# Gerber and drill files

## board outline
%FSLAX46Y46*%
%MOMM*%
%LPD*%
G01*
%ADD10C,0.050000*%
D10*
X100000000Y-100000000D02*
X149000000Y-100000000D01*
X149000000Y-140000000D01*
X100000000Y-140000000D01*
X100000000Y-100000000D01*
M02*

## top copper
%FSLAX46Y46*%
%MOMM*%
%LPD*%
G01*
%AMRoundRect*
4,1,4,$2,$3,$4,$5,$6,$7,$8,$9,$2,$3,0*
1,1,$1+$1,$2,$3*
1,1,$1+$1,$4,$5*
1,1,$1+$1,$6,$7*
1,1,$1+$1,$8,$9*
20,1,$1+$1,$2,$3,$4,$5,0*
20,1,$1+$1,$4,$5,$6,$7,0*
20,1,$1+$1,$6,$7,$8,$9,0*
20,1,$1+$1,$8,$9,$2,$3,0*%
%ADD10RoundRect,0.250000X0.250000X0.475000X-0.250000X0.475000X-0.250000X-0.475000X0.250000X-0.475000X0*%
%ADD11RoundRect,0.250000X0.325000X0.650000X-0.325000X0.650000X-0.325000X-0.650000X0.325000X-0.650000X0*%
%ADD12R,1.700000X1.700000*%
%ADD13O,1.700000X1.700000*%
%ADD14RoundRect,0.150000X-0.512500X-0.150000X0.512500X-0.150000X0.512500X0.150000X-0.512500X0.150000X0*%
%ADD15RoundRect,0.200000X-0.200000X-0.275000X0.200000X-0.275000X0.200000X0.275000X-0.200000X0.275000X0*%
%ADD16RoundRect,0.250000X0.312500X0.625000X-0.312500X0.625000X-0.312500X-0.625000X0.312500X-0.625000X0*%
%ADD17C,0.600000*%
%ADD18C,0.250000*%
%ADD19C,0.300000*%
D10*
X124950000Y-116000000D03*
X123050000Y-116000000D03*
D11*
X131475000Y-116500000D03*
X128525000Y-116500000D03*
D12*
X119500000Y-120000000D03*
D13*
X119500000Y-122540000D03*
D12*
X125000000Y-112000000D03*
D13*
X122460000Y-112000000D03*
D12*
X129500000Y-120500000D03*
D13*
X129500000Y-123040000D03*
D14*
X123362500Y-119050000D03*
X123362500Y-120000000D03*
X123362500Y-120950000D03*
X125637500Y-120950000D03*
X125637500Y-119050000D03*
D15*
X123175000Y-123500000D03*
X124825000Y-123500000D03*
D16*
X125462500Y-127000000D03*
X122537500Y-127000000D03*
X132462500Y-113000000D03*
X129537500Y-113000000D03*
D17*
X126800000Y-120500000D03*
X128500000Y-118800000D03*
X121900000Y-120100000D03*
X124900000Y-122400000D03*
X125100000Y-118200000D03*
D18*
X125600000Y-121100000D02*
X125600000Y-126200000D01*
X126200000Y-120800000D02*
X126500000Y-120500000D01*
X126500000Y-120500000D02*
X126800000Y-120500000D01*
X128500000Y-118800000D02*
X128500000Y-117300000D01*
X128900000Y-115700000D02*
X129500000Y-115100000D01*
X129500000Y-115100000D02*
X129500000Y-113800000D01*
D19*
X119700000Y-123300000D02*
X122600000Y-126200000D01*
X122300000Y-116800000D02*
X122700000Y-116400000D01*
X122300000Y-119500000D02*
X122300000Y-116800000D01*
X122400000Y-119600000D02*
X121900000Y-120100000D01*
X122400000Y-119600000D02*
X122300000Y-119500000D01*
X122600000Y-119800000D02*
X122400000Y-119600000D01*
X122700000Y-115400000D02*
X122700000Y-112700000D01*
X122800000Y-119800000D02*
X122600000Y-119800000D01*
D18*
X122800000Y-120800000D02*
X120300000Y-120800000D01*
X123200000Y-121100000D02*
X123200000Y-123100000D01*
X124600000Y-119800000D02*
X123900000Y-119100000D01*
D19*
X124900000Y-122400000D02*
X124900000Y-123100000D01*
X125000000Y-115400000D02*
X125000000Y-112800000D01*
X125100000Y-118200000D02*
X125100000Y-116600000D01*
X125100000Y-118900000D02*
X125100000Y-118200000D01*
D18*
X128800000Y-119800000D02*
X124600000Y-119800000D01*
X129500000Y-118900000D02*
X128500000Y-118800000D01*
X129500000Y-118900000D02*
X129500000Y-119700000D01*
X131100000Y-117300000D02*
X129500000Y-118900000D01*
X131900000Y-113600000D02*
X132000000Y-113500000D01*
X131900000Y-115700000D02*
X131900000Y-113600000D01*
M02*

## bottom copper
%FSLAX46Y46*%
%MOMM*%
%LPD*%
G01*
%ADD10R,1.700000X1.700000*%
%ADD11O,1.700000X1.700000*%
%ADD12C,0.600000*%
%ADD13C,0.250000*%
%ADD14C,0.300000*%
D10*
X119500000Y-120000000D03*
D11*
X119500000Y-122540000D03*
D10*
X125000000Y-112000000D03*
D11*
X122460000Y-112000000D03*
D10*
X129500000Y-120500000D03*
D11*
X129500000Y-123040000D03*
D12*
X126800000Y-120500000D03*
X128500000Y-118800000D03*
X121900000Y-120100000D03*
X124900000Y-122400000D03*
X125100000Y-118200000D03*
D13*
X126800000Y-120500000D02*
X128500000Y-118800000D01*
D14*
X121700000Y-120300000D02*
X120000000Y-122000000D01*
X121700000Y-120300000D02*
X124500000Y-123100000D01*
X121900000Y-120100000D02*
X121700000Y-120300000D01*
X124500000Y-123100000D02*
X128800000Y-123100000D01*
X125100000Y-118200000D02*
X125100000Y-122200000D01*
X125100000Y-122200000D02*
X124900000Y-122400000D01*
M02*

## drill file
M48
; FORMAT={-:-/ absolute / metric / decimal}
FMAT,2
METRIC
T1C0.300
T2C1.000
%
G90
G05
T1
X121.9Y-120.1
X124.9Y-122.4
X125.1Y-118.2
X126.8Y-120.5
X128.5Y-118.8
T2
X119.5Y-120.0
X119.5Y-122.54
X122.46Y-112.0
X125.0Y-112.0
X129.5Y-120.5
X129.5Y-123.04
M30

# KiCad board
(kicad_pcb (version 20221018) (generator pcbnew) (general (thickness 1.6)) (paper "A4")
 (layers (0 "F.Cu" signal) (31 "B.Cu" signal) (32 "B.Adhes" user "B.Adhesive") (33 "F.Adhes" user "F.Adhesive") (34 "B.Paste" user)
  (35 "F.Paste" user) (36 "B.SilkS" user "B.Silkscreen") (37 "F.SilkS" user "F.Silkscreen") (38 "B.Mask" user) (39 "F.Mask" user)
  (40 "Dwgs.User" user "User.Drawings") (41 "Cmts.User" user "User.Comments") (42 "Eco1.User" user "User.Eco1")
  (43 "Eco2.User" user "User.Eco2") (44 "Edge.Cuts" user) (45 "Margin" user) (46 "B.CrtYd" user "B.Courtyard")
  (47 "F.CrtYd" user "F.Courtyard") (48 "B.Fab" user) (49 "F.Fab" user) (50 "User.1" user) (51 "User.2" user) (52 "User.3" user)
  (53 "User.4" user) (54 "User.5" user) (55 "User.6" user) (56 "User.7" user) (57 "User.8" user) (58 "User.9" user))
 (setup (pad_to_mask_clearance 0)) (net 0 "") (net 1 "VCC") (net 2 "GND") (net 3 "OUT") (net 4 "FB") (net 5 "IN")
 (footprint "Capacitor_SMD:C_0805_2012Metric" (layer "F.Cu") (at 124 116 180)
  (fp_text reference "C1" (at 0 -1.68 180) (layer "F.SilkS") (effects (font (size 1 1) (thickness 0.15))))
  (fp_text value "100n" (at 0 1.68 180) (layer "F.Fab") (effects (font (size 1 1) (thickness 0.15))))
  (pad "1" smd roundrect (at -0.95 0 180) (size 1 1.45) (layers "F.Cu" "F.Paste" "F.Mask") (roundrect_rratio 0.25) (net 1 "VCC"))
  (pad "2" smd roundrect (at 0.95 0 180) (size 1 1.45) (layers "F.Cu" "F.Paste" "F.Mask") (roundrect_rratio 0.25) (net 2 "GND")))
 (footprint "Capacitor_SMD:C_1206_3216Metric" (layer "F.Cu") (at 130 116.5 180)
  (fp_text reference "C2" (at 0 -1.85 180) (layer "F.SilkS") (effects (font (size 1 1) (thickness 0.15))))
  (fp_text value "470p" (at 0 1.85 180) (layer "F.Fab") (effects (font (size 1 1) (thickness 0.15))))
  (pad "1" smd roundrect (at -1.475 0 180) (size 1.15 1.8) (layers "F.Cu" "F.Paste" "F.Mask") (roundrect_rratio 0.217391) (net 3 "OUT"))
  (pad "2" smd roundrect (at 1.475 0 180) (size 1.15 1.8) (layers "F.Cu" "F.Paste" "F.Mask") (roundrect_rratio 0.217391) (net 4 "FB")))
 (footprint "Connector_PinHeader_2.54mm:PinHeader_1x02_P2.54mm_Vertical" (layer "F.Cu") (at 119.5 120)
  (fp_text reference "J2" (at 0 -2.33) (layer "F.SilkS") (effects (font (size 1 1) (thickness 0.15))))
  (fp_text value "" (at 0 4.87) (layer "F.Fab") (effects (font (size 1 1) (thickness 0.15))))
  (pad "1" thru_hole rect (at 0 0) (size 1.7 1.7) (drill 1) (layers "*.Cu" "*.Mask") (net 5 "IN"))
  (pad "2" thru_hole oval (at 0 2.54) (size 1.7 1.7) (drill 1) (layers "*.Cu" "*.Mask") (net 2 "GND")))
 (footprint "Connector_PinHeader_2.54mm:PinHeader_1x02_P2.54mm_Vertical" (layer "F.Cu") (at 125 112 -90)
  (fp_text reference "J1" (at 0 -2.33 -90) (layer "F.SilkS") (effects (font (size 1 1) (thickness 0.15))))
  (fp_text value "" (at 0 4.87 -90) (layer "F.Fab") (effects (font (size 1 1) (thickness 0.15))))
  (pad "1" thru_hole rect (at 0 0 270) (size 1.7 1.7) (drill 1) (layers "*.Cu" "*.Mask") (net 1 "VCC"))
  (pad "2" thru_hole oval (at 0 2.54 270) (size 1.7 1.7) (drill 1) (layers "*.Cu" "*.Mask") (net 2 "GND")))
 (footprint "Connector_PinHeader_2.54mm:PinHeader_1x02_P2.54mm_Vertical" (layer "F.Cu") (at 129.5 120.5)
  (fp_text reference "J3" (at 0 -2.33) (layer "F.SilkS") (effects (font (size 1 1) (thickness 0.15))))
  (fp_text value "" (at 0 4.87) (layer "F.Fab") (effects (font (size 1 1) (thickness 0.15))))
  (pad "1" thru_hole rect (at 0 0) (size 1.7 1.7) (drill 1) (layers "*.Cu" "*.Mask") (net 3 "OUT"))
  (pad "2" thru_hole oval (at 0 2.54) (size 1.7 1.7) (drill 1) (layers "*.Cu" "*.Mask") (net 2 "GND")))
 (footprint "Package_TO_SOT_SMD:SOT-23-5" (layer "F.Cu") (at 124.5 120)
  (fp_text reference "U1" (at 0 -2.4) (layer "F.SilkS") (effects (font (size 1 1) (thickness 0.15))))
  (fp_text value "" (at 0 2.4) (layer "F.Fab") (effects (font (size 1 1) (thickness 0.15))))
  (pad "1" smd roundrect (at -1.1375 -0.95) (size 1.325 0.6) (layers "F.Cu" "F.Paste" "F.Mask") (roundrect_rratio 0.25) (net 3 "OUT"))
  (pad "2" smd roundrect (at -1.1375 0) (size 1.325 0.6) (layers "F.Cu" "F.Paste" "F.Mask") (roundrect_rratio 0.25) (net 2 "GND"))
  (pad "3" smd roundrect (at -1.1375 0.95) (size 1.325 0.6) (layers "F.Cu" "F.Paste" "F.Mask") (roundrect_rratio 0.25) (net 5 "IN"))
  (pad "4" smd roundrect (at 1.1375 0.95) (size 1.325 0.6) (layers "F.Cu" "F.Paste" "F.Mask") (roundrect_rratio 0.25) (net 4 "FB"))
  (pad "5" smd roundrect (at 1.1375 -0.95) (size 1.325 0.6) (layers "F.Cu" "F.Paste" "F.Mask") (roundrect_rratio 0.25) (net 1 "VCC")))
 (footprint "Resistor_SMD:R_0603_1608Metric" (layer "F.Cu") (at 124 123.5)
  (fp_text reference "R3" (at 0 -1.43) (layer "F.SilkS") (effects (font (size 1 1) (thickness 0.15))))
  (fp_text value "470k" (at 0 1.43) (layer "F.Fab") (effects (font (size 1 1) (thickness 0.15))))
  (pad "1" smd roundrect (at -0.825 0) (size 0.8 0.95) (layers "F.Cu" "F.Paste" "F.Mask") (roundrect_rratio 0.25) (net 5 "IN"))
  (pad "2" smd roundrect (at 0.825 0) (size 0.8 0.95) (layers "F.Cu" "F.Paste" "F.Mask") (roundrect_rratio 0.25) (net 1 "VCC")))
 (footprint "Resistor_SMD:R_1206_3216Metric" (layer "F.Cu") (at 124 127 180)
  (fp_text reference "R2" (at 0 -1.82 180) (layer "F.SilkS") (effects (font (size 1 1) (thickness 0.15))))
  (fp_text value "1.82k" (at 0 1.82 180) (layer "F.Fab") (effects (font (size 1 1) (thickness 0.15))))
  (pad "1" smd roundrect (at -1.4625 0 180) (size 1.125 1.75) (layers "F.Cu" "F.Paste" "F.Mask") (roundrect_rratio 0.222222) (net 4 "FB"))
  (pad "2" smd roundrect (at 1.4625 0 180) (size 1.125 1.75) (layers "F.Cu" "F.Paste" "F.Mask") (roundrect_rratio 0.222222) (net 2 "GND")))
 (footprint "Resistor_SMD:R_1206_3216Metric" (layer "F.Cu") (at 131 113 180)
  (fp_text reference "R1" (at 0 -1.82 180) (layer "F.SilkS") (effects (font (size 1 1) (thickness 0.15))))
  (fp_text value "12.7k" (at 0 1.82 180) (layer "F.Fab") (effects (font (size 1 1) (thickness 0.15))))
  (pad "1" smd roundrect (at -1.4625 0 180) (size 1.125 1.75) (layers "F.Cu" "F.Paste" "F.Mask") (roundrect_rratio 0.222222) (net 3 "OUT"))
  (pad "2" smd roundrect (at 1.4625 0 180) (size 1.125 1.75) (layers "F.Cu" "F.Paste" "F.Mask") (roundrect_rratio 0.222222) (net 4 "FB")))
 (gr_rect (start 100 100) (end 149 140) (stroke (width 0.05) (type default)) (fill none) (layer "Edge.Cuts"))
 (segment (start 125.6 121.1) (end 125.6 126.2) (width 0.25) (layer "F.Cu") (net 4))
 (segment (start 126.2 120.8) (end 126.5 120.5) (width 0.25) (layer "F.Cu") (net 4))
 (segment (start 126.5 120.5) (end 126.8 120.5) (width 0.25) (layer "F.Cu") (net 4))
 (segment (start 128.5 118.8) (end 128.5 117.3) (width 0.25) (layer "F.Cu") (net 4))
 (segment (start 128.9 115.7) (end 129.5 115.1) (width 0.25) (layer "F.Cu") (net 4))
 (segment (start 129.5 115.1) (end 129.5 113.8) (width 0.25) (layer "F.Cu") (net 4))
 (via (at 126.8 120.5) (size 0.6) (drill 0.3) (layers "F.Cu" "B.Cu") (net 4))
 (via (at 128.5 118.8) (size 0.6) (drill 0.3) (layers "F.Cu" "B.Cu") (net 4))
 (segment (start 119.7 123.3) (end 122.6 126.2) (width 0.3) (layer "F.Cu") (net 2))
 (segment (start 122.3 116.8) (end 122.7 116.4) (width 0.3) (layer "F.Cu") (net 2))
 (segment (start 122.3 119.5) (end 122.3 116.8) (width 0.3) (layer "F.Cu") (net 2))
 (segment (start 122.4 119.6) (end 121.9 120.1) (width 0.3) (layer "F.Cu") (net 2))
 (segment (start 122.4 119.6) (end 122.3 119.5) (width 0.3) (layer "F.Cu") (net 2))
 (segment (start 122.6 119.8) (end 122.4 119.6) (width 0.3) (layer "F.Cu") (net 2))
 (segment (start 122.7 115.4) (end 122.7 112.7) (width 0.3) (layer "F.Cu") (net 2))
 (segment (start 122.8 119.8) (end 122.6 119.8) (width 0.3) (layer "F.Cu") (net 2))
 (segment (start 126.8 120.5) (end 128.5 118.8) (width 0.25) (layer "B.Cu") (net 4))
 (via (at 121.9 120.1) (size 0.6) (drill 0.3) (layers "F.Cu" "B.Cu") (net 2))
 (segment (start 121.7 120.3) (end 120 122) (width 0.3) (layer "B.Cu") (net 2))
 (segment (start 121.7 120.3) (end 124.5 123.1) (width 0.3) (layer "B.Cu") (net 2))
 (segment (start 121.9 120.1) (end 121.7 120.3) (width 0.3) (layer "B.Cu") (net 2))
 (segment (start 122.8 120.8) (end 120.3 120.8) (width 0.25) (layer "F.Cu") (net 5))
 (segment (start 123.2 121.1) (end 123.2 123.1) (width 0.25) (layer "F.Cu") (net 5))
 (segment (start 124.5 123.1) (end 128.8 123.1) (width 0.3) (layer "B.Cu") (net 2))
 (segment (start 124.6 119.8) (end 123.9 119.1) (width 0.25) (layer "F.Cu") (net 3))
 (segment (start 124.9 122.4) (end 124.9 123.1) (width 0.3) (layer "F.Cu") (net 1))
 (segment (start 125 115.4) (end 125 112.8) (width 0.3) (layer "F.Cu") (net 1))
 (segment (start 125.1 118.2) (end 125.1 116.6) (width 0.3) (layer "F.Cu") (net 1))
 (segment (start 125.1 118.9) (end 125.1 118.2) (width 0.3) (layer "F.Cu") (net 1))
 (segment (start 128.8 119.8) (end 124.6 119.8) (width 0.25) (layer "F.Cu") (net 3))
 (segment (start 129.5 118.9) (end 128.5 118.8) (width 0.25) (layer "F.Cu") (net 3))
 (segment (start 129.5 118.9) (end 129.5 119.7) (width 0.25) (layer "F.Cu") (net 3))
 (segment (start 131.1 117.3) (end 129.5 118.9) (width 0.25) (layer "F.Cu") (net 3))
 (segment (start 131.9 113.6) (end 132 113.5) (width 0.25) (layer "F.Cu") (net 3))
 (segment (start 131.9 115.7) (end 131.9 113.6) (width 0.25) (layer "F.Cu") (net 3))
 (via (at 124.9 122.4) (size 0.6) (drill 0.3) (layers "F.Cu" "B.Cu") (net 1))
 (via (at 125.1 118.2) (size 0.6) (drill 0.3) (layers "F.Cu" "B.Cu") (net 1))
 (segment (start 125.1 118.2) (end 125.1 122.2) (width 0.3) (layer "B.Cu") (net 1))
 (segment (start 125.1 122.2) (end 124.9 122.4) (width 0.3) (layer "B.Cu") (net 1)))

